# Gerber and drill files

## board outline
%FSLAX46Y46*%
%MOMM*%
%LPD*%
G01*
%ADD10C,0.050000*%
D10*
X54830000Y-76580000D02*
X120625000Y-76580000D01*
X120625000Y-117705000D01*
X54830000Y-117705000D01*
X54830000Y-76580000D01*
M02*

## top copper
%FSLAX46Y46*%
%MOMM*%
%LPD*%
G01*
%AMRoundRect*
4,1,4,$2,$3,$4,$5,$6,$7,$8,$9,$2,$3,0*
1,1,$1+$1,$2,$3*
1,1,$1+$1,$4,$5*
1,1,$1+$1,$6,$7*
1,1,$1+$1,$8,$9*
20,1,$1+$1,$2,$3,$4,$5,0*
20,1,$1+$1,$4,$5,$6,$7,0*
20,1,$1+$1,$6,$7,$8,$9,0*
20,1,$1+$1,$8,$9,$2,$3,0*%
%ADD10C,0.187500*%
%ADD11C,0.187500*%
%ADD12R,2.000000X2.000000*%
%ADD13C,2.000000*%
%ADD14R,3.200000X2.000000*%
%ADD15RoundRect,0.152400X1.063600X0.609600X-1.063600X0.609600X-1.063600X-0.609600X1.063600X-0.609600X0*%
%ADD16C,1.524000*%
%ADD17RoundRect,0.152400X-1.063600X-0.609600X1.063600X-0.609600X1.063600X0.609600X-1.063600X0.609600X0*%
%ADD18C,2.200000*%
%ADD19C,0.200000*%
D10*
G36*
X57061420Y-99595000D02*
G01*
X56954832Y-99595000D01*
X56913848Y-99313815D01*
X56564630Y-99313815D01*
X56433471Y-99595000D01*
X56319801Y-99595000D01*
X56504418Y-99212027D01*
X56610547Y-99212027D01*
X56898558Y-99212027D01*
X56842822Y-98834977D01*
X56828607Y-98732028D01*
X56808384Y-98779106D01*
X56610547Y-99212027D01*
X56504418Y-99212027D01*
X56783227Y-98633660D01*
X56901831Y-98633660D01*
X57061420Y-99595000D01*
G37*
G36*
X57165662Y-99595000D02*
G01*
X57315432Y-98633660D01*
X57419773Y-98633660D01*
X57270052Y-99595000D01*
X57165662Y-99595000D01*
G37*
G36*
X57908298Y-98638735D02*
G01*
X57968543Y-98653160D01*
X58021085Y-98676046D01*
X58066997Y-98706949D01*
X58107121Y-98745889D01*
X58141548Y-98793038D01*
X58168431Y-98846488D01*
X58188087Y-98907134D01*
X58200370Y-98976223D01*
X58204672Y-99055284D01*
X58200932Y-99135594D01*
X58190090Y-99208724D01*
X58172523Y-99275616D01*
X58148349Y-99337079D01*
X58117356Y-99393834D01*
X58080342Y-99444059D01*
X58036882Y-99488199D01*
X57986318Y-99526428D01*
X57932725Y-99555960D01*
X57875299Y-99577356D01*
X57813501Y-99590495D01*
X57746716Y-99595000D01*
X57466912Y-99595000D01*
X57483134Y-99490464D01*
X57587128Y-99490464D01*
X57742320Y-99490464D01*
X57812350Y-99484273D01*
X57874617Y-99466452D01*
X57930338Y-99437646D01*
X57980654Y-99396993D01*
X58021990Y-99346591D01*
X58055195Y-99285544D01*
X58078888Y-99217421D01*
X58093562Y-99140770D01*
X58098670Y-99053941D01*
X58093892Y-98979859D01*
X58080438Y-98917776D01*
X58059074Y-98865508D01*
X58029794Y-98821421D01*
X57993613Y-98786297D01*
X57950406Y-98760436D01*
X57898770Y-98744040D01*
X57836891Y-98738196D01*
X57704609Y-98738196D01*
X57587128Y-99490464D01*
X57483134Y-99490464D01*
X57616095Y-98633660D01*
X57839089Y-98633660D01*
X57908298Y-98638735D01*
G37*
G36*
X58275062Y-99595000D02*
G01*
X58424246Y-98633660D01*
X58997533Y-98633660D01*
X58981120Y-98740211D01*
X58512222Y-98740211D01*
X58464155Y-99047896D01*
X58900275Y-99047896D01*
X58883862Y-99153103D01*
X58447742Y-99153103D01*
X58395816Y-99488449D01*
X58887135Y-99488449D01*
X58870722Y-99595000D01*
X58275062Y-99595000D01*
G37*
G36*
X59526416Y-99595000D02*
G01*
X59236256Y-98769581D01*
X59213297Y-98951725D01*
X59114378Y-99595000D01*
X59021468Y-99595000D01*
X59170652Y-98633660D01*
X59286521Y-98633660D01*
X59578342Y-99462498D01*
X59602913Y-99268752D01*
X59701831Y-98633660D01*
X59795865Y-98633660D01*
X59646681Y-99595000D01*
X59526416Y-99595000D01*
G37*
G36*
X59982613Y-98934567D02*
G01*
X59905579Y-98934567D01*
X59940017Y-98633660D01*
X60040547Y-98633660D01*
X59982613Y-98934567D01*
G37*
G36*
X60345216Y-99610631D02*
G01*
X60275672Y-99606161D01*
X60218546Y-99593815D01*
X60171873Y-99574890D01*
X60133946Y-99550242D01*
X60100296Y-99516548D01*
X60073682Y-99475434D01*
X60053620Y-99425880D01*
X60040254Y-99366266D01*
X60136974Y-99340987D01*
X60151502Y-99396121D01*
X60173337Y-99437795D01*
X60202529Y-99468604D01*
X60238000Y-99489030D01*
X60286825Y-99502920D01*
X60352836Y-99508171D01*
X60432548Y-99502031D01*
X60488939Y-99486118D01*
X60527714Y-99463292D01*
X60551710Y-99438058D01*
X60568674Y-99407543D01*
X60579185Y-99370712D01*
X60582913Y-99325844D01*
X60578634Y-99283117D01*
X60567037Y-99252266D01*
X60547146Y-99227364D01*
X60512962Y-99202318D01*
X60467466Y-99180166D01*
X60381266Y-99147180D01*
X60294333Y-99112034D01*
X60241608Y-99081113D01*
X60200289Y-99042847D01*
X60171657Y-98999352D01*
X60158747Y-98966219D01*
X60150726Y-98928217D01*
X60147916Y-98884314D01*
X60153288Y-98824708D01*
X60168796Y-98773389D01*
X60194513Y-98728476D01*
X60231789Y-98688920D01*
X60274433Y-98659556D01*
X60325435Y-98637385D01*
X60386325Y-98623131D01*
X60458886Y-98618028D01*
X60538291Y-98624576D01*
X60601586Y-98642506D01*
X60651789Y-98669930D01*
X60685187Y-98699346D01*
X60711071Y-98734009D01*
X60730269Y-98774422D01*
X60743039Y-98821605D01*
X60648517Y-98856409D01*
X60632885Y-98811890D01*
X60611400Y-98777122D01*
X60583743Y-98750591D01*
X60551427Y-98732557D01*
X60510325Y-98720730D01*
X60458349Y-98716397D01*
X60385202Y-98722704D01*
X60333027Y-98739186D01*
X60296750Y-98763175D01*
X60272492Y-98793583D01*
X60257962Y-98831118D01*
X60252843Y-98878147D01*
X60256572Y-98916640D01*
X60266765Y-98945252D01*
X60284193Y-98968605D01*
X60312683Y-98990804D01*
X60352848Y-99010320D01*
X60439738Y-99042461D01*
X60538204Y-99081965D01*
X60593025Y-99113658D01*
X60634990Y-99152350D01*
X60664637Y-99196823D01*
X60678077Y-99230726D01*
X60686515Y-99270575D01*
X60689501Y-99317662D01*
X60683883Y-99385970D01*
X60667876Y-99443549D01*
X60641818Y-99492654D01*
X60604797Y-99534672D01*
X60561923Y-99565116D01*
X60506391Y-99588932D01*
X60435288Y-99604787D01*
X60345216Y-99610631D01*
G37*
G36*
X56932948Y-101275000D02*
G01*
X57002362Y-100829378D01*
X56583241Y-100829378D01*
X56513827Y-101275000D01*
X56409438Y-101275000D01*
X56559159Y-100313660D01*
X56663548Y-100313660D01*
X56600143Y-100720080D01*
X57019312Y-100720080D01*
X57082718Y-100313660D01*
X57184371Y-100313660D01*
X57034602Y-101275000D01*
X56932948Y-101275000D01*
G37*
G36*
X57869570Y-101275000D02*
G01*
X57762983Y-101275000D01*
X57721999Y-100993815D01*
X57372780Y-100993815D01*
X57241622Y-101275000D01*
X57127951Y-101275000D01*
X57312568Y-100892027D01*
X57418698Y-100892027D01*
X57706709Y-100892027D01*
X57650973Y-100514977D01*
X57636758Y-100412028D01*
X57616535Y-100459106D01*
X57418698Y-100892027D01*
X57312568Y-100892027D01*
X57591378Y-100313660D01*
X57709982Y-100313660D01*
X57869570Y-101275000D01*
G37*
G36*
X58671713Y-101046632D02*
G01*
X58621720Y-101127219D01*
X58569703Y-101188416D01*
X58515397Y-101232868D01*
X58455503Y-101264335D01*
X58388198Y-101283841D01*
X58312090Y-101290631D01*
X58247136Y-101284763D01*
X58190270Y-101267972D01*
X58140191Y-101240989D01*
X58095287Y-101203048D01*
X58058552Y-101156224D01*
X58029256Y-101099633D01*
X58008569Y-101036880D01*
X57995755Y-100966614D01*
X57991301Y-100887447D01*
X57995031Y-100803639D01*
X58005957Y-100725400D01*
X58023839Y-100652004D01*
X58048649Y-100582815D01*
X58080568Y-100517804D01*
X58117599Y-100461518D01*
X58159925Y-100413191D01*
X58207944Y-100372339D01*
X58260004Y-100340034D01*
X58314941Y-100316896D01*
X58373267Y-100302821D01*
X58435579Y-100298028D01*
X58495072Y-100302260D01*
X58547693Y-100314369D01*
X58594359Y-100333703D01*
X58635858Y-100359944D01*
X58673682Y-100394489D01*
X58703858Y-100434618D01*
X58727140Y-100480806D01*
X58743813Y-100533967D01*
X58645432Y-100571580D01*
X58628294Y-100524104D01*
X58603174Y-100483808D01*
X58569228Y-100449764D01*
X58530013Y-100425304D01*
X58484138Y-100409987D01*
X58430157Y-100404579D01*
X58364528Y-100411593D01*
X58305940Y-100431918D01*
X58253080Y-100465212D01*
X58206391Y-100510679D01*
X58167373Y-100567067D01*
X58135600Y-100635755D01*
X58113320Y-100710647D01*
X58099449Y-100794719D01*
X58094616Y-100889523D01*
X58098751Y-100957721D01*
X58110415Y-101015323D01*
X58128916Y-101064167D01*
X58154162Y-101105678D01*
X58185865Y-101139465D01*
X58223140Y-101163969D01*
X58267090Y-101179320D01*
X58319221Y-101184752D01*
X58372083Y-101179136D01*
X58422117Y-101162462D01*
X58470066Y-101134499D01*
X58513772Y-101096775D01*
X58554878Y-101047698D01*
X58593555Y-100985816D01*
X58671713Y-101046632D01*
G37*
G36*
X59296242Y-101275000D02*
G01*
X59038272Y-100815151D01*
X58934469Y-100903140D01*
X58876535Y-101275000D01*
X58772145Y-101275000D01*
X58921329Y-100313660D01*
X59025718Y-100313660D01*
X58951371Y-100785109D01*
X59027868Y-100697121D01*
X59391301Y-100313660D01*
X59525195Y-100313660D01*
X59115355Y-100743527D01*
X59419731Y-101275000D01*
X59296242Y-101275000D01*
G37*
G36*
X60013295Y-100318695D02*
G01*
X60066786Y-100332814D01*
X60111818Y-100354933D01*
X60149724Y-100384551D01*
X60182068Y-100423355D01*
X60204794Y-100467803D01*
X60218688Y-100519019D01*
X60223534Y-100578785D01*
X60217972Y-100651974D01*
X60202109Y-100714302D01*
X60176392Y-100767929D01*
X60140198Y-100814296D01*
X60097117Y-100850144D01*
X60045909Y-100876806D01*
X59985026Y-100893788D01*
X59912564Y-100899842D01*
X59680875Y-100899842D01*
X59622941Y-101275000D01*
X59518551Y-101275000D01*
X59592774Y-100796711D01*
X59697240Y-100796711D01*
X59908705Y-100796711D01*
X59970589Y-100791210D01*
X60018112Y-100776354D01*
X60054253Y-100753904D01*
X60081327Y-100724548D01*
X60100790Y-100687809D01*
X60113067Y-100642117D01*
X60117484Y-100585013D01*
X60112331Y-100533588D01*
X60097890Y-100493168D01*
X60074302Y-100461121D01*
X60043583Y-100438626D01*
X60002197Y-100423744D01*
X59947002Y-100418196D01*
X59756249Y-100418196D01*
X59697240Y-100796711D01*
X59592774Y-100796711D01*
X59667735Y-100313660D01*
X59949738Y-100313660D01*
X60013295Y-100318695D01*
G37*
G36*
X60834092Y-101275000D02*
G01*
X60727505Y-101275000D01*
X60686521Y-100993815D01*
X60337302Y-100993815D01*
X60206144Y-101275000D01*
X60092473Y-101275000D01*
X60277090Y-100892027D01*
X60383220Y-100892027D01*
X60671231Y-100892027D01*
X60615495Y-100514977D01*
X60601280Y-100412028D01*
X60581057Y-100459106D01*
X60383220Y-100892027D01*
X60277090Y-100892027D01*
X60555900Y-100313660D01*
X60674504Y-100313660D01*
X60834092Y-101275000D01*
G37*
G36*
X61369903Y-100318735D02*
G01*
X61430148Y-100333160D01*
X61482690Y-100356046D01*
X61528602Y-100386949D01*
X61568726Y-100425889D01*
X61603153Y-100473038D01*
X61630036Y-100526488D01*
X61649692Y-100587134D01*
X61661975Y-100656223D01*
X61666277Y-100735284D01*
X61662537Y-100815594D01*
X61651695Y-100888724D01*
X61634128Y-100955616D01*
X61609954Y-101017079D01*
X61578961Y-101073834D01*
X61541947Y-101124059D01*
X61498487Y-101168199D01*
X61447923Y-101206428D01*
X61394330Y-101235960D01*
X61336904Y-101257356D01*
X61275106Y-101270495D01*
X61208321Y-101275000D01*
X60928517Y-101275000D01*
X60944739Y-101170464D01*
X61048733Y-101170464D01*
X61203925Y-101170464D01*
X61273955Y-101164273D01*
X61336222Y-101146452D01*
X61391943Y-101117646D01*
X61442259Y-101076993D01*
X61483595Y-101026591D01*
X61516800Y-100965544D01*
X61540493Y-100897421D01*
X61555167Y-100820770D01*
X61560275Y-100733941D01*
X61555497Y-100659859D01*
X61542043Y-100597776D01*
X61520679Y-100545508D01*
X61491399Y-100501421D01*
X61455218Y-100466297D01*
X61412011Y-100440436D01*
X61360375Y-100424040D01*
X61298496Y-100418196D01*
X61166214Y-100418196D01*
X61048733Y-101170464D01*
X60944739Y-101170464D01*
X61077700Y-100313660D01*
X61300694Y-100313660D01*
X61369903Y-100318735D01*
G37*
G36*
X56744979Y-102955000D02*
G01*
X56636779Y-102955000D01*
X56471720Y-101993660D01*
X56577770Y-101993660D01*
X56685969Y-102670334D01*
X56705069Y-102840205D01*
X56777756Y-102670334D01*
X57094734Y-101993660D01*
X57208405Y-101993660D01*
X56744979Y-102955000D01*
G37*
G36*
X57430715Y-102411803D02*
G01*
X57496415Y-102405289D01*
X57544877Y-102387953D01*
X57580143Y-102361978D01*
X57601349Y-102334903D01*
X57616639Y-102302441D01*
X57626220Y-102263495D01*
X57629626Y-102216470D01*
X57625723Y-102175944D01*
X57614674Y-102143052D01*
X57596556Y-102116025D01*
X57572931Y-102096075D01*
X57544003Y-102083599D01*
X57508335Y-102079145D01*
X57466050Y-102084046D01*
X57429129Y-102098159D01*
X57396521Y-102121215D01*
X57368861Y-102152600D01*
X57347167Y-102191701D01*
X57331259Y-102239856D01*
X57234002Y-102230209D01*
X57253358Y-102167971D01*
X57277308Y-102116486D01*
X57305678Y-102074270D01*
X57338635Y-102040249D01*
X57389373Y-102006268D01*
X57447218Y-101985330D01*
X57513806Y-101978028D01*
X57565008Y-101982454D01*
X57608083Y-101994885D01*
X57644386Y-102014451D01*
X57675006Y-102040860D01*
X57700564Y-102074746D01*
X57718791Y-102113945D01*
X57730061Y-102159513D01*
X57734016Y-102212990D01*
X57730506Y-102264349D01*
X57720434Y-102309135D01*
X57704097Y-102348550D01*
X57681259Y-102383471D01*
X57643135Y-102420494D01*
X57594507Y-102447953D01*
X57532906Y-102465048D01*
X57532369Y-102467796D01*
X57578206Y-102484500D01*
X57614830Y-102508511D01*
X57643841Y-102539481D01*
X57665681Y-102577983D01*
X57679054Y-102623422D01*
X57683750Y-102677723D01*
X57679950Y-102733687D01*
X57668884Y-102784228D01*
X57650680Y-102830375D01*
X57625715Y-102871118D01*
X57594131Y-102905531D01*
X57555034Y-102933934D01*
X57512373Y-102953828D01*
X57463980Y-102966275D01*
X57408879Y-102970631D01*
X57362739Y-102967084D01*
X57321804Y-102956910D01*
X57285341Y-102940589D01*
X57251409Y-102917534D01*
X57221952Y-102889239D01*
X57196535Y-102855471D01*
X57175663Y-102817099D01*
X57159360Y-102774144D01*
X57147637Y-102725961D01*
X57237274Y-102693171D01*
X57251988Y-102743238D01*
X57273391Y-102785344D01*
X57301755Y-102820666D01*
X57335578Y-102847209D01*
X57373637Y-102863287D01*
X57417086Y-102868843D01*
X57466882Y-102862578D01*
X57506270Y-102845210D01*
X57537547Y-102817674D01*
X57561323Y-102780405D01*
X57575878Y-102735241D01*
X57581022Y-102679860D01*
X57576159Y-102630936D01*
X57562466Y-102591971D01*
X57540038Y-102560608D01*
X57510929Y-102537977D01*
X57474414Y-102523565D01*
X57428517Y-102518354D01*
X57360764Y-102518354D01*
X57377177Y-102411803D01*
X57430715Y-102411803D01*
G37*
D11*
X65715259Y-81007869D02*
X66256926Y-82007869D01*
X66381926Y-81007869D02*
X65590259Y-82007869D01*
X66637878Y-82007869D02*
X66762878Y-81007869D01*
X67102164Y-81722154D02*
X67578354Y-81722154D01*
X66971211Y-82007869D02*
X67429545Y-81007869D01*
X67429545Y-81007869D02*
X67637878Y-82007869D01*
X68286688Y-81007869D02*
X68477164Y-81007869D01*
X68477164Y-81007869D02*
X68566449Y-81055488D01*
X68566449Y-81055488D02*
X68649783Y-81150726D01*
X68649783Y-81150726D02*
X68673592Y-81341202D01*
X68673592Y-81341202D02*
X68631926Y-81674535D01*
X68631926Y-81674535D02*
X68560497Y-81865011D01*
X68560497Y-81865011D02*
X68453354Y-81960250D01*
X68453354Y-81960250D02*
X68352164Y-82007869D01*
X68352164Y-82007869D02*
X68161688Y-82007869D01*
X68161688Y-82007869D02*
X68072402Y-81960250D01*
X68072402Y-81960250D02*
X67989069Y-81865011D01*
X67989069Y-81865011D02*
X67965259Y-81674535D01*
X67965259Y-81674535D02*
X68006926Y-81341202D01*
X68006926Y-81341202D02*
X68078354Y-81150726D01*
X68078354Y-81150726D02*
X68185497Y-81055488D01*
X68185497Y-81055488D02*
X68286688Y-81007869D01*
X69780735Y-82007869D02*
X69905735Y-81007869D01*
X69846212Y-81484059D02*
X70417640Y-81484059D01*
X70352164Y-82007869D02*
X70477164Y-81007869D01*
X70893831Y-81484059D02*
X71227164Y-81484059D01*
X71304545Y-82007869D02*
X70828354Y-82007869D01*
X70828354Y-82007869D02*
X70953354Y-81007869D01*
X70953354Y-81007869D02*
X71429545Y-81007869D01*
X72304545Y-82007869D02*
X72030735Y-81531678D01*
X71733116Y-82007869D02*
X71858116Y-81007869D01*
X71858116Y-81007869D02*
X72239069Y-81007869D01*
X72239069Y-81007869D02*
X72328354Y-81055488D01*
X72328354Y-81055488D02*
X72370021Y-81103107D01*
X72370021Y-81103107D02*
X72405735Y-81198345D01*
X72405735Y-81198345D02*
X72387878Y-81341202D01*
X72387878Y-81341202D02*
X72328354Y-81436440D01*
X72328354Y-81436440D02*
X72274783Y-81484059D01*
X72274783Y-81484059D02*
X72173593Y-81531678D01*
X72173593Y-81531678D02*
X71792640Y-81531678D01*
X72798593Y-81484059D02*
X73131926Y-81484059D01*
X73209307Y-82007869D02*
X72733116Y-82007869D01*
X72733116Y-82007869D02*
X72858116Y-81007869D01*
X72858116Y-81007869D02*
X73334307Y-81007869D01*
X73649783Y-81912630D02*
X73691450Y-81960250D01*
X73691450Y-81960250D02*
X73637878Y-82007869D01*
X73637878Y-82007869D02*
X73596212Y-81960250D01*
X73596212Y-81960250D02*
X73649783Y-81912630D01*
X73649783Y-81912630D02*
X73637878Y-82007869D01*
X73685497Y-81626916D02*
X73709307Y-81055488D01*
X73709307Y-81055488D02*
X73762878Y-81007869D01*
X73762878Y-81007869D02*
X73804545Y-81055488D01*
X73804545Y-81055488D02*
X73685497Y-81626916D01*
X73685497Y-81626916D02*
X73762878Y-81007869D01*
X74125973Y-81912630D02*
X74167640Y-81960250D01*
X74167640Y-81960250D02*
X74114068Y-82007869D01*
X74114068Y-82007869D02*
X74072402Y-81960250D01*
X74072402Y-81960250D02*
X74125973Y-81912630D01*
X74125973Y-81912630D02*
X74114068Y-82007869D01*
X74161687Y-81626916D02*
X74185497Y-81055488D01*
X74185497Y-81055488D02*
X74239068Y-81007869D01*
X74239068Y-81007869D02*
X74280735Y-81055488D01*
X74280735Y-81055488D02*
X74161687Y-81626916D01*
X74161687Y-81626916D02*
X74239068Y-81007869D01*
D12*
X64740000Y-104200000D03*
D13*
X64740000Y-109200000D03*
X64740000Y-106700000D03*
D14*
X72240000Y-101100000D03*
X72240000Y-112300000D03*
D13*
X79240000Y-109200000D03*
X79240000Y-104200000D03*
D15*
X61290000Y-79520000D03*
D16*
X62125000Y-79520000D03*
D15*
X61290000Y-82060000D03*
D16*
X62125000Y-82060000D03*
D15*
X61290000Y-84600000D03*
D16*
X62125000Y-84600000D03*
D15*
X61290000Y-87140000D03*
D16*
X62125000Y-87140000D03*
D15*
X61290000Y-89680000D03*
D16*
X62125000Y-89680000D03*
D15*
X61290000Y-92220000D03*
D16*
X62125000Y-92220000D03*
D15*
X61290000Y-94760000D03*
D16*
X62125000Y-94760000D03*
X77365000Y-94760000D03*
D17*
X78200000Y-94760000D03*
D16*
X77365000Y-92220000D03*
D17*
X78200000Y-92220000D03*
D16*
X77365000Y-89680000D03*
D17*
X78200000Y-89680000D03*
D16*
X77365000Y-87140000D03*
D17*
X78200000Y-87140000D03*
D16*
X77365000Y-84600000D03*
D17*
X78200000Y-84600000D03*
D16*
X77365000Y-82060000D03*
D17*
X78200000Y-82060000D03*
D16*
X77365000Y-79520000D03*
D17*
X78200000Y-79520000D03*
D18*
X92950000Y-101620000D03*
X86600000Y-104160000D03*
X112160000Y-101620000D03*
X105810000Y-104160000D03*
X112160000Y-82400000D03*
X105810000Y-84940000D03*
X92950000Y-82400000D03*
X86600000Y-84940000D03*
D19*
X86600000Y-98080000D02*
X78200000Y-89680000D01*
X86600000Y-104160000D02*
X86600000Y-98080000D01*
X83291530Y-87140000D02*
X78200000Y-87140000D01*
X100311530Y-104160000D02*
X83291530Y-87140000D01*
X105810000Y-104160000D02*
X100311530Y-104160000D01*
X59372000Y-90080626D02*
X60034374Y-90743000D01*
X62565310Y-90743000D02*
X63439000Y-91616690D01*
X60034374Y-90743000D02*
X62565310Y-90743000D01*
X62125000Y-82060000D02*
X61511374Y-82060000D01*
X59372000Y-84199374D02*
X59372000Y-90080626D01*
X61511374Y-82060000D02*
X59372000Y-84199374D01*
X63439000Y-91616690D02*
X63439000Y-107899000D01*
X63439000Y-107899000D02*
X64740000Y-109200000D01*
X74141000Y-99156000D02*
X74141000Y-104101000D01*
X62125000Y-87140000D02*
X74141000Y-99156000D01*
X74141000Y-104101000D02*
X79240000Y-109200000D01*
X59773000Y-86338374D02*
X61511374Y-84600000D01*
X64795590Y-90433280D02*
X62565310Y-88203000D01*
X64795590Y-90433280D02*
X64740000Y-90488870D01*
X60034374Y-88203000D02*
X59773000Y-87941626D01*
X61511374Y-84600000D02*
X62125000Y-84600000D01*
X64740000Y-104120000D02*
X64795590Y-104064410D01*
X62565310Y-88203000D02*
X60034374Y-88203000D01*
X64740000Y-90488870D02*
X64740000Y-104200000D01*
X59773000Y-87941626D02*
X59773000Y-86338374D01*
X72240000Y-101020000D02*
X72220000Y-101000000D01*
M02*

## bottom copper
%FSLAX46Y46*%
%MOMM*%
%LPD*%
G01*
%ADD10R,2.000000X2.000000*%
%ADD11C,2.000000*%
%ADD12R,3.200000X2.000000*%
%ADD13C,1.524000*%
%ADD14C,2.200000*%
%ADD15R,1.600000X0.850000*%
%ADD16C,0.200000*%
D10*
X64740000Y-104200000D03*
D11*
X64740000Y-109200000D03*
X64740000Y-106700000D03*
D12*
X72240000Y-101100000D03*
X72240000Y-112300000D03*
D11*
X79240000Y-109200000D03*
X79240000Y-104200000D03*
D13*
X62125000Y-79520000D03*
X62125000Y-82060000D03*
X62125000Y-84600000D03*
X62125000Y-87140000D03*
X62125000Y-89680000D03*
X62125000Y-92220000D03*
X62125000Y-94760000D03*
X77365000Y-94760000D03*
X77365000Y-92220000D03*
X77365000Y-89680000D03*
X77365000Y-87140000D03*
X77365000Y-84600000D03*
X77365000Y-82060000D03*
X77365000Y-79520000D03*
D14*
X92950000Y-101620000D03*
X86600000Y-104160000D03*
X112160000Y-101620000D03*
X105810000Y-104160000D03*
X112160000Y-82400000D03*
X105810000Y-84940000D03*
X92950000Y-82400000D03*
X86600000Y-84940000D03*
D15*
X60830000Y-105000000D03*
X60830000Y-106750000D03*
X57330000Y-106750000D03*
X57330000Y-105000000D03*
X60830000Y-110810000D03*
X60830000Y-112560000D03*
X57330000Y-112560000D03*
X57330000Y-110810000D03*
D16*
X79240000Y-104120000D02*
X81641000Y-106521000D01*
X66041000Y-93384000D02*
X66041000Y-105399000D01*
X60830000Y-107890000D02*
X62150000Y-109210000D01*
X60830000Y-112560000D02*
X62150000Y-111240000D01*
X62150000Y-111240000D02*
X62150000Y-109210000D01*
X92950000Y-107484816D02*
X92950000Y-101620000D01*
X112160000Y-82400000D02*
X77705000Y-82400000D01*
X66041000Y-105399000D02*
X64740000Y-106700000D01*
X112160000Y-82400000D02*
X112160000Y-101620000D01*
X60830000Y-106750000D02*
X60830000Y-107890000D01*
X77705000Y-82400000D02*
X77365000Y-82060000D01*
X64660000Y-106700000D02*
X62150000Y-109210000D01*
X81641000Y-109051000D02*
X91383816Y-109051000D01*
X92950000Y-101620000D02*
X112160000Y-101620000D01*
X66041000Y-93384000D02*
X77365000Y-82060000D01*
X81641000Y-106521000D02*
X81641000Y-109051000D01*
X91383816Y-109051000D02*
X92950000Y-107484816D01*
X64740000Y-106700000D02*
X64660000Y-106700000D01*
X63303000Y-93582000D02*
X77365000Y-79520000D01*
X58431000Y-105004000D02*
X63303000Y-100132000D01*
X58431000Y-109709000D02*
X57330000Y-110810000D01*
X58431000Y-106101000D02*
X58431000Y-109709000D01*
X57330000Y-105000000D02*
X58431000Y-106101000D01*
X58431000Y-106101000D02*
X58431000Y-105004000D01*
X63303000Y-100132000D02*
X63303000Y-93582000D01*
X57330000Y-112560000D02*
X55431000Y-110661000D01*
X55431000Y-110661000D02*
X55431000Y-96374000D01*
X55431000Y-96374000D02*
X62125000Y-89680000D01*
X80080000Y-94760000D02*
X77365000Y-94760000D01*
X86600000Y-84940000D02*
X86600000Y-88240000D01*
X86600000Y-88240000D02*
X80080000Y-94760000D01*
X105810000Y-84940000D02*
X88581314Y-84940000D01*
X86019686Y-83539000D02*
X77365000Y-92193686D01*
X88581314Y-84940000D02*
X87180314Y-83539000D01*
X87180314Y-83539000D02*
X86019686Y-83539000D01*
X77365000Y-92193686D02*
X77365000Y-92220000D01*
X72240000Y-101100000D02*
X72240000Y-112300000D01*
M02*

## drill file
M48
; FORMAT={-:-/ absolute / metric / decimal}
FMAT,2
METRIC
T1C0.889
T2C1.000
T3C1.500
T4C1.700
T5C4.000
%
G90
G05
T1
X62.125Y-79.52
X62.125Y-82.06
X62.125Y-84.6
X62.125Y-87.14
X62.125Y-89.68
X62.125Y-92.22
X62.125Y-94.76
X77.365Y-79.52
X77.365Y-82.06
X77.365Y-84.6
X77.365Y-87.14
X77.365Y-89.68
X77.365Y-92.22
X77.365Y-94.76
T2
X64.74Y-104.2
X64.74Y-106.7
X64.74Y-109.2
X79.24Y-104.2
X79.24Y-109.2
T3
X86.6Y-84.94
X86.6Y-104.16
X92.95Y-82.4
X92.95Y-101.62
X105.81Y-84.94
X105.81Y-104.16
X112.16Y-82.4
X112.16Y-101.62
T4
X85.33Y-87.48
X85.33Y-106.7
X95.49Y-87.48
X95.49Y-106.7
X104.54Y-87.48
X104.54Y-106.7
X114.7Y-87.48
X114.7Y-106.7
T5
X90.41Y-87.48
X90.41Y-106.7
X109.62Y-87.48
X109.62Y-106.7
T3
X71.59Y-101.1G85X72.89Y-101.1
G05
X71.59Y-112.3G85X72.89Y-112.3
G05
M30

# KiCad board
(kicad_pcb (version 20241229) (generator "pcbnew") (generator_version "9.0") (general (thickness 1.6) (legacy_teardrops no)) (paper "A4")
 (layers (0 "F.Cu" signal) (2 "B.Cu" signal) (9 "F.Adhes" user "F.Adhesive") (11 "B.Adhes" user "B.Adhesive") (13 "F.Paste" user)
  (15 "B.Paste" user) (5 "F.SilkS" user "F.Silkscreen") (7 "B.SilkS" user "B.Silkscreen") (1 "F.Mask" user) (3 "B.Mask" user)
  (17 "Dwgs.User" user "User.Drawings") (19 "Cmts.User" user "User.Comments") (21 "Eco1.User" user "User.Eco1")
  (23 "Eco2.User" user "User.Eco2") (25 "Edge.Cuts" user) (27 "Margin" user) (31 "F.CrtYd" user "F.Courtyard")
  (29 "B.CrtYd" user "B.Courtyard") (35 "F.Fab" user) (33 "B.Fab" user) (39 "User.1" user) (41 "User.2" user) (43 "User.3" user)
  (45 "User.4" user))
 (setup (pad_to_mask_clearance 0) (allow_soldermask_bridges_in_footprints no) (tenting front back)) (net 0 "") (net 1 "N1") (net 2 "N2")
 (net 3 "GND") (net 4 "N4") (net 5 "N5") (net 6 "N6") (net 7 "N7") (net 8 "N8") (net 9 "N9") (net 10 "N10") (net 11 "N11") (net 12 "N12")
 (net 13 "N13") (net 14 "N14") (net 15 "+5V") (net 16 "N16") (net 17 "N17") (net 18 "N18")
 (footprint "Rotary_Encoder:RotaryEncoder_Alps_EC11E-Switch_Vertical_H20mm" (layer "F.Cu") (at 64.74 104.2)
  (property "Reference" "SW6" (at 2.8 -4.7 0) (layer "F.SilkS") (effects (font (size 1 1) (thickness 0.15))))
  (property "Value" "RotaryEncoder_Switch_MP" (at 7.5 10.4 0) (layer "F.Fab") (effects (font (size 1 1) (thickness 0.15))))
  (pad "A" thru_hole rect (at 0 0) (size 2 2) (drill 1) (layers "*.Cu" "*.Mask") (remove_unused_layers no) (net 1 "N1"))
  (pad "B" thru_hole circle (at 0 5) (size 2 2) (drill 1) (layers "*.Cu" "*.Mask") (remove_unused_layers no) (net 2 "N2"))
  (pad "C" thru_hole circle (at 0 2.5) (size 2 2) (drill 1) (layers "*.Cu" "*.Mask") (remove_unused_layers no) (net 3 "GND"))
  (pad "MP" thru_hole rect (at 7.5 -3.1) (size 3.2 2) (drill oval 2.8 1.5) (layers "*.Cu" "*.Mask") (remove_unused_layers no) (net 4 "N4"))
  (pad "MP" thru_hole rect (at 7.5 8.1) (size 3.2 2) (drill oval 2.8 1.5) (layers "*.Cu" "*.Mask") (remove_unused_layers no) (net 4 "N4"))
  (pad "S1" thru_hole circle (at 14.5 5) (size 2 2) (drill 1) (layers "*.Cu" "*.Mask") (remove_unused_layers no) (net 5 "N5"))
  (pad "S2" thru_hole circle (at 14.5 0) (size 2 2) (drill 1) (layers "*.Cu" "*.Mask") (remove_unused_layers no) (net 3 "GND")))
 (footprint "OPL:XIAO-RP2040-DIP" (layer "F.Cu") (at 69.745 87.14)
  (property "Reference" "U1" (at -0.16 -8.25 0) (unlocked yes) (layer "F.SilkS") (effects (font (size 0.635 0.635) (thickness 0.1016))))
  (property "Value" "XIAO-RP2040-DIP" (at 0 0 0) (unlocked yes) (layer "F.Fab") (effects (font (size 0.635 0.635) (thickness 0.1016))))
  (pad "1" smd roundrect (at -8.455 -7.62 180) (size 2.432 1.524) (layers "F.Cu" "F.Mask") (roundrect_rratio 0.1) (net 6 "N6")
   (thermal_bridge_angle 45))
  (pad "1" thru_hole circle (at -7.62 -7.62 180) (size 1.524 1.524) (drill 0.889) (layers "*.Cu" "*.Mask") (remove_unused_layers no)
   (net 6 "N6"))
  (pad "2" smd roundrect (at -8.455 -5.08 180) (size 2.432 1.524) (layers "F.Cu" "F.Mask") (roundrect_rratio 0.1) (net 2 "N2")
   (thermal_bridge_angle 45))
  (pad "2" thru_hole circle (at -7.62 -5.08 180) (size 1.524 1.524) (drill 0.889) (layers "*.Cu" "*.Mask") (remove_unused_layers no)
   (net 2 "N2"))
  (pad "3" smd roundrect (at -8.455 -2.54 180) (size 2.432 1.524) (layers "F.Cu" "F.Mask") (roundrect_rratio 0.1) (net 1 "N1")
   (thermal_bridge_angle 45))
  (pad "3" thru_hole circle (at -7.62 -2.54 180) (size 1.524 1.524) (drill 0.889) (layers "*.Cu" "*.Mask") (remove_unused_layers no)
   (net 1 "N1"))
  (pad "4" smd roundrect (at -8.455 0 180) (size 2.432 1.524) (layers "F.Cu" "F.Mask") (roundrect_rratio 0.1) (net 5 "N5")
   (thermal_bridge_angle 45))
  (pad "4" thru_hole circle (at -7.62 0 180) (size 1.524 1.524) (drill 0.889) (layers "*.Cu" "*.Mask") (remove_unused_layers no)
   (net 5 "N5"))
  (pad "5" smd roundrect (at -8.455 2.54 180) (size 2.432 1.524) (layers "F.Cu" "F.Mask") (roundrect_rratio 0.1) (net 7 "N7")
   (thermal_bridge_angle 45))
  (pad "5" thru_hole circle (at -7.62 2.54 180) (size 1.524 1.524) (drill 0.889) (layers "*.Cu" "*.Mask") (remove_unused_layers no)
   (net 7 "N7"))
  (pad "6" smd roundrect (at -8.455 5.08 180) (size 2.432 1.524) (layers "F.Cu" "F.Mask") (roundrect_rratio 0.1) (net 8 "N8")
   (thermal_bridge_angle 45))
  (pad "6" thru_hole circle (at -7.62 5.08 180) (size 1.524 1.524) (drill 0.889) (layers "*.Cu" "*.Mask") (remove_unused_layers no)
   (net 8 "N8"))
  (pad "7" smd roundrect (at -8.455 7.62 180) (size 2.432 1.524) (layers "F.Cu" "F.Mask") (roundrect_rratio 0.1) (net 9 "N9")
   (thermal_bridge_angle 45))
  (pad "7" thru_hole circle (at -7.62 7.62 180) (size 1.524 1.524) (drill 0.889) (layers "*.Cu" "*.Mask") (remove_unused_layers no)
   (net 9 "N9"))
  (pad "8" thru_hole circle (at 7.62 7.62) (size 1.524 1.524) (drill 0.889) (layers "*.Cu" "*.Mask") (remove_unused_layers no)
   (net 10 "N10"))
  (pad "8" smd roundrect (at 8.455 7.62) (size 2.432 1.524) (layers "F.Cu" "F.Mask") (roundrect_rratio 0.1) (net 10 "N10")
   (thermal_bridge_angle 45))
  (pad "9" thru_hole circle (at 7.62 5.08) (size 1.524 1.524) (drill 0.889) (layers "*.Cu" "*.Mask") (remove_unused_layers no)
   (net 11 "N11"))
  (pad "9" smd roundrect (at 8.455 5.08) (size 2.432 1.524) (layers "F.Cu" "F.Mask") (roundrect_rratio 0.1) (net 11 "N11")
   (thermal_bridge_angle 45))
  (pad "10" thru_hole circle (at 7.62 2.54) (size 1.524 1.524) (drill 0.889) (layers "*.Cu" "*.Mask") (remove_unused_layers no)
   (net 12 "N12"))
  (pad "10" smd roundrect (at 8.455 2.54) (size 2.432 1.524) (layers "F.Cu" "F.Mask") (roundrect_rratio 0.1) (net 12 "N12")
   (thermal_bridge_angle 45))
  (pad "11" thru_hole circle (at 7.62 0) (size 1.524 1.524) (drill 0.889) (layers "*.Cu" "*.Mask") (remove_unused_layers no) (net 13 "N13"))
  (pad "11" smd roundrect (at 8.455 0) (size 2.432 1.524) (layers "F.Cu" "F.Mask") (roundrect_rratio 0.1) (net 13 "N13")
   (thermal_bridge_angle 45))
  (pad "12" thru_hole circle (at 7.62 -2.54) (size 1.524 1.524) (drill 0.889) (layers "*.Cu" "*.Mask") (remove_unused_layers no)
   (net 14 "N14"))
  (pad "12" smd roundrect (at 8.455 -2.54) (size 2.432 1.524) (layers "F.Cu" "F.Mask") (roundrect_rratio 0.1) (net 14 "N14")
   (thermal_bridge_angle 45))
  (pad "13" thru_hole circle (at 7.62 -5.08) (size 1.524 1.524) (drill 0.889) (layers "*.Cu" "*.Mask") (remove_unused_layers no)
   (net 3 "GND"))
  (pad "13" smd roundrect (at 8.455 -5.08) (size 2.432 1.524) (layers "F.Cu" "F.Mask") (roundrect_rratio 0.1) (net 3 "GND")
   (thermal_bridge_angle 45))
  (pad "14" thru_hole circle (at 7.62 -7.62) (size 1.524 1.524) (drill 0.889) (layers "*.Cu" "*.Mask") (remove_unused_layers no)
   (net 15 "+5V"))
  (pad "14" smd roundrect (at 8.455 -7.62) (size 2.432 1.524) (layers "F.Cu" "F.Mask") (roundrect_rratio 0.1) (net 15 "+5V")
   (thermal_bridge_angle 45)))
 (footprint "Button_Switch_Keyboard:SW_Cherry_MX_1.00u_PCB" (layer "F.Cu") (at 92.95 101.62)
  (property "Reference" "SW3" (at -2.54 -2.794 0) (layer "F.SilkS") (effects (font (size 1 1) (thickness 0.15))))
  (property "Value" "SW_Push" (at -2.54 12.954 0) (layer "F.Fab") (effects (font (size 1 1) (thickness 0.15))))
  (pad "" np_thru_hole circle (at -7.62 5.08) (size 1.7 1.7) (drill 1.7) (layers "*.Cu" "*.Mask"))
  (pad "" np_thru_hole circle (at -2.54 5.08) (size 4 4) (drill 4) (layers "*.Cu" "*.Mask"))
  (pad "" np_thru_hole circle (at 2.54 5.08) (size 1.7 1.7) (drill 1.7) (layers "*.Cu" "*.Mask"))
  (pad "1" thru_hole circle (at 0 0) (size 2.2 2.2) (drill 1.5) (layers "*.Cu" "*.Mask") (remove_unused_layers no) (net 3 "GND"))
  (pad "2" thru_hole circle (at -6.35 2.54) (size 2.2 2.2) (drill 1.5) (layers "*.Cu" "*.Mask") (remove_unused_layers no) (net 12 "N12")))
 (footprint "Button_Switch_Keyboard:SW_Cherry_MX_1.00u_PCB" (layer "F.Cu") (at 112.16 101.62)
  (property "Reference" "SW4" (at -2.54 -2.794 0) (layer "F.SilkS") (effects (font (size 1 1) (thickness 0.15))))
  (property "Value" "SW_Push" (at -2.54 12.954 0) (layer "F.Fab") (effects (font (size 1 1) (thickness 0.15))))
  (pad "" np_thru_hole circle (at -7.62 5.08) (size 1.7 1.7) (drill 1.7) (layers "*.Cu" "*.Mask"))
  (pad "" np_thru_hole circle (at -2.54 5.08) (size 4 4) (drill 4) (layers "*.Cu" "*.Mask"))
  (pad "" np_thru_hole circle (at 2.54 5.08) (size 1.7 1.7) (drill 1.7) (layers "*.Cu" "*.Mask"))
  (pad "1" thru_hole circle (at 0 0) (size 2.2 2.2) (drill 1.5) (layers "*.Cu" "*.Mask") (remove_unused_layers no) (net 3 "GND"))
  (pad "2" thru_hole circle (at -6.35 2.54) (size 2.2 2.2) (drill 1.5) (layers "*.Cu" "*.Mask") (remove_unused_layers no) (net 13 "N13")))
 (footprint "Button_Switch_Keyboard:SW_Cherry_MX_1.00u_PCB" (layer "F.Cu") (at 112.16 82.4)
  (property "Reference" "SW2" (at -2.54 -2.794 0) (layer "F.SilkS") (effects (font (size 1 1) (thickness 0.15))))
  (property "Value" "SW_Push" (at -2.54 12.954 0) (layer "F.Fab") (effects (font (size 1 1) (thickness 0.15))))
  (pad "" np_thru_hole circle (at -7.62 5.08) (size 1.7 1.7) (drill 1.7) (layers "*.Cu" "*.Mask"))
  (pad "" np_thru_hole circle (at -2.54 5.08) (size 4 4) (drill 4) (layers "*.Cu" "*.Mask"))
  (pad "" np_thru_hole circle (at 2.54 5.08) (size 1.7 1.7) (drill 1.7) (layers "*.Cu" "*.Mask"))
  (pad "1" thru_hole circle (at 0 0) (size 2.2 2.2) (drill 1.5) (layers "*.Cu" "*.Mask") (remove_unused_layers no) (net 3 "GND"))
  (pad "2" thru_hole circle (at -6.35 2.54) (size 2.2 2.2) (drill 1.5) (layers "*.Cu" "*.Mask") (remove_unused_layers no) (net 11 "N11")))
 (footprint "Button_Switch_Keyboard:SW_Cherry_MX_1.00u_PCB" (layer "F.Cu") (at 92.95 82.4)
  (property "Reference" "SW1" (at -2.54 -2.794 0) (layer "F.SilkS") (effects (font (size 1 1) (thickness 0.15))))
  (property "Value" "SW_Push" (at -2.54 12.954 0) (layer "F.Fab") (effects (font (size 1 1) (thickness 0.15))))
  (pad "" np_thru_hole circle (at -7.62 5.08) (size 1.7 1.7) (drill 1.7) (layers "*.Cu" "*.Mask"))
  (pad "" np_thru_hole circle (at -2.54 5.08) (size 4 4) (drill 4) (layers "*.Cu" "*.Mask"))
  (pad "" np_thru_hole circle (at 2.54 5.08) (size 1.7 1.7) (drill 1.7) (layers "*.Cu" "*.Mask"))
  (pad "1" thru_hole circle (at 0 0) (size 2.2 2.2) (drill 1.5) (layers "*.Cu" "*.Mask") (remove_unused_layers no) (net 3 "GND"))
  (pad "2" thru_hole circle (at -6.35 2.54) (size 2.2 2.2) (drill 1.5) (layers "*.Cu" "*.Mask") (remove_unused_layers no) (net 10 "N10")))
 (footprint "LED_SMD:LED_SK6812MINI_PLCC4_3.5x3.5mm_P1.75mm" (layer "B.Cu") (at 59.08 105.875 180)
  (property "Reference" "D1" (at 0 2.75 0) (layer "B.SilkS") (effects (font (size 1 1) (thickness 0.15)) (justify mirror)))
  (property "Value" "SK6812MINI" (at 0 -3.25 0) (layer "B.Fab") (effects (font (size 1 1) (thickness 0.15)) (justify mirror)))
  (pad "1" smd rect (at -1.75 0.875 180) (size 1.6 0.85) (layers "B.Cu" "B.Mask" "B.Paste") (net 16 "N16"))
  (pad "2" smd rect (at -1.75 -0.875 180) (size 1.6 0.85) (layers "B.Cu" "B.Mask" "B.Paste") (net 3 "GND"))
  (pad "3" smd rect (at 1.75 -0.875 180) (size 1.6 0.85) (layers "B.Cu" "B.Mask" "B.Paste") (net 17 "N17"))
  (pad "4" smd rect (at 1.75 0.875 180) (size 1.6 0.85) (layers "B.Cu" "B.Mask" "B.Paste") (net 15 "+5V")))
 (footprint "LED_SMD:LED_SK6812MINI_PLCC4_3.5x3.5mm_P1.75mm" (layer "B.Cu") (at 59.08 111.685 180)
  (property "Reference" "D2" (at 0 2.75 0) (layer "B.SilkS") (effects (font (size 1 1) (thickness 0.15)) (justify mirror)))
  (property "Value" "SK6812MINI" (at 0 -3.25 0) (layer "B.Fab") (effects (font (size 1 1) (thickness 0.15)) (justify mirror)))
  (pad "1" smd rect (at -1.75 0.875 180) (size 1.6 0.85) (layers "B.Cu" "B.Mask" "B.Paste") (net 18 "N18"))
  (pad "2" smd rect (at -1.75 -0.875 180) (size 1.6 0.85) (layers "B.Cu" "B.Mask" "B.Paste") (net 3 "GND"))
  (pad "3" smd rect (at 1.75 -0.875 180) (size 1.6 0.85) (layers "B.Cu" "B.Mask" "B.Paste") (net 7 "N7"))
  (pad "4" smd rect (at 1.75 0.875 180) (size 1.6 0.85) (layers "B.Cu" "B.Mask" "B.Paste") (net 15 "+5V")))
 (gr_rect (start 54.83 76.58) (end 120.625 117.705) (stroke (width 0.05) (type default)) (fill no) (layer "Edge.Cuts"))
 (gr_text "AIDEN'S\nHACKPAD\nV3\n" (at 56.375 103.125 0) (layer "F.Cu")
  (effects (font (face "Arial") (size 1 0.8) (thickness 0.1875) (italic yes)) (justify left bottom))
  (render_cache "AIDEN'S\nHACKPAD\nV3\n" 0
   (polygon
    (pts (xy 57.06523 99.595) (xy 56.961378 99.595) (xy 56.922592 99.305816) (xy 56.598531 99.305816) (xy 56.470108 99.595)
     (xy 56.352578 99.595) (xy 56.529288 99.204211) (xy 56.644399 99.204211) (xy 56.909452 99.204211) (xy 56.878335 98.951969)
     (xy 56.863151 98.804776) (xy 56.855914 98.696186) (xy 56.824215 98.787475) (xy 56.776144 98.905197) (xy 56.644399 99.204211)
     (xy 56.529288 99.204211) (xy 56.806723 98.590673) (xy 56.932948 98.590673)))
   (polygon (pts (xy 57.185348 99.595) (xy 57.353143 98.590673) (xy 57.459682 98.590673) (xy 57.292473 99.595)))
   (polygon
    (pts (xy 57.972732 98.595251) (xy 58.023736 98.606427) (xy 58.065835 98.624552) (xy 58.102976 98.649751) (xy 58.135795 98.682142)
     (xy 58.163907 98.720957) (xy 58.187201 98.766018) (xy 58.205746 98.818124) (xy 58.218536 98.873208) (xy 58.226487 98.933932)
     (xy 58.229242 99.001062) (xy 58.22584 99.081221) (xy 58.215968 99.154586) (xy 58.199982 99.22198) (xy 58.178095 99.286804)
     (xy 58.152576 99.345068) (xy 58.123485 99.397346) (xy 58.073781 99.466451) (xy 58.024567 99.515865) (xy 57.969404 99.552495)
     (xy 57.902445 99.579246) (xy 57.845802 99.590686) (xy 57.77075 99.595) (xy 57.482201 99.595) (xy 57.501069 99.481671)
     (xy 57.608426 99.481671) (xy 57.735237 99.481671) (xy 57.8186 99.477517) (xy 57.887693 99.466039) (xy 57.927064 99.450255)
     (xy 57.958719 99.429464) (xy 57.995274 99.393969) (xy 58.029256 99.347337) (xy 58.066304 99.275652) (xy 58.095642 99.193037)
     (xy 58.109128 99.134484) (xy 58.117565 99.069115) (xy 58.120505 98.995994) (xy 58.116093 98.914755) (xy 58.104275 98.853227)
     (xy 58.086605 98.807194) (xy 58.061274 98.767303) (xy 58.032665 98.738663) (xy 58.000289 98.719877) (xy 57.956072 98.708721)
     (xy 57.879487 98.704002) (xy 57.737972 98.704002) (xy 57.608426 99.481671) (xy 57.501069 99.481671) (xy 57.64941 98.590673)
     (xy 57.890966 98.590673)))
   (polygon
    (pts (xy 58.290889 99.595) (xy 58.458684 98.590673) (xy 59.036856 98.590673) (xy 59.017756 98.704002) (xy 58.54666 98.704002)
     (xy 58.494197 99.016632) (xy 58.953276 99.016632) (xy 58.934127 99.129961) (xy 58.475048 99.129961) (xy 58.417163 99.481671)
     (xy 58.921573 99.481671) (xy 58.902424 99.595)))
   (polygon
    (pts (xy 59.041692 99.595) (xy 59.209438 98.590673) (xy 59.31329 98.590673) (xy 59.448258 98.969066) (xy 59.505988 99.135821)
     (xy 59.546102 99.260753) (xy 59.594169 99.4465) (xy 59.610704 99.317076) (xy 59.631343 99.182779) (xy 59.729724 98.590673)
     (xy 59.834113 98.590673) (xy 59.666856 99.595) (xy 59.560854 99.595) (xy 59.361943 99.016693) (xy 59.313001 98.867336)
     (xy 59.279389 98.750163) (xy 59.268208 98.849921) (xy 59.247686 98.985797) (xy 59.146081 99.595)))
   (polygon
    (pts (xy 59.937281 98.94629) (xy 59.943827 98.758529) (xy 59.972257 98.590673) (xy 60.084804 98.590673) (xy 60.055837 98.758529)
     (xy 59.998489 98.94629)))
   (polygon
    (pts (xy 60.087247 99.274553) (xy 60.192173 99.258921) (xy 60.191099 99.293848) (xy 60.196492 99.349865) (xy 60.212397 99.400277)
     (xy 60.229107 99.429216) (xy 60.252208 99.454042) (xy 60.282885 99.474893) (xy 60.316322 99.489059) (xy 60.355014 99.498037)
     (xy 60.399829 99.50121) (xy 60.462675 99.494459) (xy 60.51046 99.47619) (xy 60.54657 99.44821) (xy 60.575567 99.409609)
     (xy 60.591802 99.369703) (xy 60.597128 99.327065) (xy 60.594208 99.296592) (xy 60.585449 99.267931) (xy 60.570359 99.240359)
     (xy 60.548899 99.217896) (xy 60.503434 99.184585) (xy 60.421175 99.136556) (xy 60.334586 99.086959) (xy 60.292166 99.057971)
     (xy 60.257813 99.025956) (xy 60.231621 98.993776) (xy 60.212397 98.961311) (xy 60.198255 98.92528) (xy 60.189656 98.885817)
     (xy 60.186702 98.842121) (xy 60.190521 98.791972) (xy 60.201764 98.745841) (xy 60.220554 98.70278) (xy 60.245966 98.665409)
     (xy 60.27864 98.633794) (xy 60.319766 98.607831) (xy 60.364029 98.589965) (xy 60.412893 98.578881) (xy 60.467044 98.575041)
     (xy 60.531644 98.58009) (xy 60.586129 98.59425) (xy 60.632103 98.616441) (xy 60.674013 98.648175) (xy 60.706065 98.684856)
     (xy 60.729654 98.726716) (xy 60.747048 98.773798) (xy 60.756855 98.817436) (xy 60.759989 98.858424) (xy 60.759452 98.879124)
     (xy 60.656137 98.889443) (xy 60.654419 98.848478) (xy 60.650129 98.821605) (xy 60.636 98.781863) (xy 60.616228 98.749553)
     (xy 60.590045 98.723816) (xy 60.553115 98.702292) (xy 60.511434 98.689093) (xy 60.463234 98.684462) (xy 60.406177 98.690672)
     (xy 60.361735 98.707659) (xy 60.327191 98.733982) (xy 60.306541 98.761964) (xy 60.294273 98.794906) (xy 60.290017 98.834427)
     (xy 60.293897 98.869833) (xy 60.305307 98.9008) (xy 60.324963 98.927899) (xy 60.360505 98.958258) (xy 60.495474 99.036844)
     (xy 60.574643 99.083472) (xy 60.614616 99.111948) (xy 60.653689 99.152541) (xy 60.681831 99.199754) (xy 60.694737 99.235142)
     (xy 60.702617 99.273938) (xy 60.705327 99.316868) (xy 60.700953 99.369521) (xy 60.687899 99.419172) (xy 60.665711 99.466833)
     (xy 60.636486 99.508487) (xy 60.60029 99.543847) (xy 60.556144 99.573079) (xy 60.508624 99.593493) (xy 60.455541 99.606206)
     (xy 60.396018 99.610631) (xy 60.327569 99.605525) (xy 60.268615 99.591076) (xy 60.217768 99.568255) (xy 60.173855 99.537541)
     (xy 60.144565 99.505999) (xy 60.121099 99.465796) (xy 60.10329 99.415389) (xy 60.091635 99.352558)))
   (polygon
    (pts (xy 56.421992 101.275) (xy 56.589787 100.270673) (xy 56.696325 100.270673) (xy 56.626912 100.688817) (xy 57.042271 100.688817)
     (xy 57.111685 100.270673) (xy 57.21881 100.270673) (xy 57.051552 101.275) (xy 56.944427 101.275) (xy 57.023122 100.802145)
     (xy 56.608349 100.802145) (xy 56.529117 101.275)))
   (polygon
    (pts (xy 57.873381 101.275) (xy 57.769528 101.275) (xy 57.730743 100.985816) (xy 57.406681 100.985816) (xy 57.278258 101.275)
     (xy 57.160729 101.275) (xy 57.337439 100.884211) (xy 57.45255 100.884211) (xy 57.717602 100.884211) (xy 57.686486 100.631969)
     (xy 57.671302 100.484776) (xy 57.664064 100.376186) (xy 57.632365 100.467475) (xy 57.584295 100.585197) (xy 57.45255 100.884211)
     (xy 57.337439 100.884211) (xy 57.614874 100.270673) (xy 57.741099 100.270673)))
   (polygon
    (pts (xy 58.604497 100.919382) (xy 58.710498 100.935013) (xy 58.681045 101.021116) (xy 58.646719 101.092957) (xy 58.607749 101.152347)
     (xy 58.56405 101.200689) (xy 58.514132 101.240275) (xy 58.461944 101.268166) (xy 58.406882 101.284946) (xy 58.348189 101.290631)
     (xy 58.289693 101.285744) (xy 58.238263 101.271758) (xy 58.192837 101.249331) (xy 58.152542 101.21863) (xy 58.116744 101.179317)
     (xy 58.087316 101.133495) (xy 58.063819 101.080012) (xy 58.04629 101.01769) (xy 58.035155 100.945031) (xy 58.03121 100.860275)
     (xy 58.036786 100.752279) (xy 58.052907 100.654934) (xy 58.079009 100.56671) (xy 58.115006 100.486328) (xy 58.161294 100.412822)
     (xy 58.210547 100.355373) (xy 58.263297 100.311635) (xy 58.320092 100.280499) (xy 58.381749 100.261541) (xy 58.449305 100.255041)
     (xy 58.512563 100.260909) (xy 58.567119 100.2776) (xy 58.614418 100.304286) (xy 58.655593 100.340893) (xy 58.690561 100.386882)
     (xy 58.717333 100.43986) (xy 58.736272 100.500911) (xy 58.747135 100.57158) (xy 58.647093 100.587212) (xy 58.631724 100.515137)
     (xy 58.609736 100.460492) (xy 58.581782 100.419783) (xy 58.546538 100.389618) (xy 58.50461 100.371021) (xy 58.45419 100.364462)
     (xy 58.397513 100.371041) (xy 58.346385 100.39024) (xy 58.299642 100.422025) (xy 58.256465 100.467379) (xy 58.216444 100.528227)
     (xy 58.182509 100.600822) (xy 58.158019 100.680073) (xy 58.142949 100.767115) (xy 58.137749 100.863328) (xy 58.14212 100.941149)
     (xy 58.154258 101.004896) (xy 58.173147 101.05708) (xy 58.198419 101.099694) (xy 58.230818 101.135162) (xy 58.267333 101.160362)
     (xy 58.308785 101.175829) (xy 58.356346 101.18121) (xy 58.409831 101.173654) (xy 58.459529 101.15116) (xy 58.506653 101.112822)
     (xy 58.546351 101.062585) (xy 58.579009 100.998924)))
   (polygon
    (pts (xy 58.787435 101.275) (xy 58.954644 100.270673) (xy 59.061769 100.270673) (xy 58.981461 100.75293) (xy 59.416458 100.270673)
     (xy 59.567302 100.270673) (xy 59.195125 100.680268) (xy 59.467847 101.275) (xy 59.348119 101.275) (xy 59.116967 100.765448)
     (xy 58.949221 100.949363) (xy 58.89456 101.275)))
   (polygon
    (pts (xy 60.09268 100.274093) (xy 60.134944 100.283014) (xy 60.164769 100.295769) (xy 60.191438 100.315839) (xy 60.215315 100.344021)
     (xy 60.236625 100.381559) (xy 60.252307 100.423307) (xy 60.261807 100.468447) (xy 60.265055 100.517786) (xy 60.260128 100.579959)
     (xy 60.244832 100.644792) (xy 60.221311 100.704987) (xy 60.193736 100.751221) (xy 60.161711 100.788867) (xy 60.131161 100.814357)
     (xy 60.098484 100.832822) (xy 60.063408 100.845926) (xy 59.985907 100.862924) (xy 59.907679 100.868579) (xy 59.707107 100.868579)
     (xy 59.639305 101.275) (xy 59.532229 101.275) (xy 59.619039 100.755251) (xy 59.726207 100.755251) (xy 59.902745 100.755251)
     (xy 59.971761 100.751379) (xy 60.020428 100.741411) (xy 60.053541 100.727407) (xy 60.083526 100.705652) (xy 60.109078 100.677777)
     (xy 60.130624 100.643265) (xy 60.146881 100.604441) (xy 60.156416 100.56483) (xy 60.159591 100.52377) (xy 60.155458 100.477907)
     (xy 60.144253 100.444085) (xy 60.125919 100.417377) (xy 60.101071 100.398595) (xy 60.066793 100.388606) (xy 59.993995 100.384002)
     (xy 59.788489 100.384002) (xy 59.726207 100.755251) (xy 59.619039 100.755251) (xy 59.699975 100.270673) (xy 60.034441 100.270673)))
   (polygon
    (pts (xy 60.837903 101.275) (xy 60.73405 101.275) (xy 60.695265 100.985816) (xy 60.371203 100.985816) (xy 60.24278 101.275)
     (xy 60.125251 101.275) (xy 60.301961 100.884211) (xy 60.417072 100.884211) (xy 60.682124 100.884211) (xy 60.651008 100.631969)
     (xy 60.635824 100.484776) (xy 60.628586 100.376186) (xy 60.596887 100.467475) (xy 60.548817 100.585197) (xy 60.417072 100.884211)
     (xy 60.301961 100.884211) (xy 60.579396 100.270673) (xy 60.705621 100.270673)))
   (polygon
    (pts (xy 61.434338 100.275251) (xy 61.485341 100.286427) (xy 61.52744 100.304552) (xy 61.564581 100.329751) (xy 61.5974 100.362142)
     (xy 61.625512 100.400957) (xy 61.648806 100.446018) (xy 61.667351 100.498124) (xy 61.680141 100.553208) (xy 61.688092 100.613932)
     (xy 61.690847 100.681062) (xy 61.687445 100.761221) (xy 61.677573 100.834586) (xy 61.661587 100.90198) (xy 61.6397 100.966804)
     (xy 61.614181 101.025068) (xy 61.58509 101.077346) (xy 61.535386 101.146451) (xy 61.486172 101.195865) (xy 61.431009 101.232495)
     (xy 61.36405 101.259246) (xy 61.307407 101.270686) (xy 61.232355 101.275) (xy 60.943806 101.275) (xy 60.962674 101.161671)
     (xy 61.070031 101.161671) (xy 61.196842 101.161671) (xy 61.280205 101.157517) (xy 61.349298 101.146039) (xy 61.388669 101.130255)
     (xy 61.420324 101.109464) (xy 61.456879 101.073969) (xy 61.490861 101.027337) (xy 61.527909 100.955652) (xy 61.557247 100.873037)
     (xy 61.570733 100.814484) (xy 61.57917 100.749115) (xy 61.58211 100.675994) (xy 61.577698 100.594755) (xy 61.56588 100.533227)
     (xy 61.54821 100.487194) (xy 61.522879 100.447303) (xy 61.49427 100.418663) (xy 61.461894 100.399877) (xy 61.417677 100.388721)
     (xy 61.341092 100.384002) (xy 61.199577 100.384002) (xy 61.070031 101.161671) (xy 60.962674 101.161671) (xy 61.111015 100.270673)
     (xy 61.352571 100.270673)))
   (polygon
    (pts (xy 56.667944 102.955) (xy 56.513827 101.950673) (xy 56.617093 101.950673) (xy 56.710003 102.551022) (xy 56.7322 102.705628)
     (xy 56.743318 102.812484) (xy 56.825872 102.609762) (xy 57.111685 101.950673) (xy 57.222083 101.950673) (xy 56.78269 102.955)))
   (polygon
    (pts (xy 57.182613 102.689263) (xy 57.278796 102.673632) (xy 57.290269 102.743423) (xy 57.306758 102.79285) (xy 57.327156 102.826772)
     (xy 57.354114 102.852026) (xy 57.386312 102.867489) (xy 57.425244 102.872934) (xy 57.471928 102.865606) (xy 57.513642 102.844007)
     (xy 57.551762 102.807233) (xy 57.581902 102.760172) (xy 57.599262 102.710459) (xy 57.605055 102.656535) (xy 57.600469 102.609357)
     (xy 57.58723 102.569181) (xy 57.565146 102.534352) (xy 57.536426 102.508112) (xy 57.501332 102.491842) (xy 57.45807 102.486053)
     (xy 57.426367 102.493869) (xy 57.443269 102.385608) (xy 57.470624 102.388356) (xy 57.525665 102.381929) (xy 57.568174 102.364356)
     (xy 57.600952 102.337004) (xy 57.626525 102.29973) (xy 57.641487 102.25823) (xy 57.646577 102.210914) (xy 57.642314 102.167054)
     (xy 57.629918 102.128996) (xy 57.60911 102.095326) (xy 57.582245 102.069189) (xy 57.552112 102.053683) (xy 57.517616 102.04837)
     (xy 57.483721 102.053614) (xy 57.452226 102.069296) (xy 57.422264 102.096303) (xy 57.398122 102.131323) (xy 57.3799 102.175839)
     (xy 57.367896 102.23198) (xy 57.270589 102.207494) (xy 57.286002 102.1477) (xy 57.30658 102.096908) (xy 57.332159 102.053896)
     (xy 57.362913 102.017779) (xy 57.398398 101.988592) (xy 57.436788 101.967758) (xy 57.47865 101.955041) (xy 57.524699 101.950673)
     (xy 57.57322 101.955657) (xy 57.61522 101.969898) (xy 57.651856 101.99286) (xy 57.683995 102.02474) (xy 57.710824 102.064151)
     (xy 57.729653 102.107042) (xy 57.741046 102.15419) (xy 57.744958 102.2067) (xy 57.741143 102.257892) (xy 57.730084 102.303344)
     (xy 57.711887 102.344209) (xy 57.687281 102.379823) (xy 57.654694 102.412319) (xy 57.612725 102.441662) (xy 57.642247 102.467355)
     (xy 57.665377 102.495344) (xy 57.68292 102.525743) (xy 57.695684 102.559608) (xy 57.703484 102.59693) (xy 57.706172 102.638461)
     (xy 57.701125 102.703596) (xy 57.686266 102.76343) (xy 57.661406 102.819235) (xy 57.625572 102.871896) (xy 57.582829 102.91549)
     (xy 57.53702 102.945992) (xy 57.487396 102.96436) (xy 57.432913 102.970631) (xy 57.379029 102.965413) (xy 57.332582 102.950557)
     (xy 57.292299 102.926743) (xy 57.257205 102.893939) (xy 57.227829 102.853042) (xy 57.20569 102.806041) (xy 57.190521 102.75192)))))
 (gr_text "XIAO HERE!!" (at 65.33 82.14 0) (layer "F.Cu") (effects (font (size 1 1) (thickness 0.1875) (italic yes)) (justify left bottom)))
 (segment (start 79.24 104.12) (end 81.641 106.521) (width 0.2) (layer "B.Cu") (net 3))
 (segment (start 66.041 93.384) (end 66.041 105.399) (width 0.2) (layer "B.Cu") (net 3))
 (segment (start 60.83 107.89) (end 62.15 109.21) (width 0.2) (layer "B.Cu") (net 3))
 (segment (start 60.83 112.56) (end 62.15 111.24) (width 0.2) (layer "B.Cu") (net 3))
 (segment (start 62.15 111.24) (end 62.15 109.21) (width 0.2) (layer "B.Cu") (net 3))
 (segment (start 92.95 107.484816) (end 92.95 101.62) (width 0.2) (layer "B.Cu") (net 3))
 (segment (start 112.16 82.4) (end 77.705 82.4) (width 0.2) (layer "B.Cu") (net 3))
 (segment (start 66.041 105.399) (end 64.74 106.7) (width 0.2) (layer "B.Cu") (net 3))
 (segment (start 112.16 82.4) (end 112.16 101.62) (width 0.2) (layer "B.Cu") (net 3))
 (segment (start 60.83 106.75) (end 60.83 107.89) (width 0.2) (layer "B.Cu") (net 3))
 (segment (start 77.705 82.4) (end 77.365 82.06) (width 0.2) (layer "B.Cu") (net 3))
 (segment (start 64.66 106.7) (end 62.15 109.21) (width 0.2) (layer "B.Cu") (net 3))
 (segment (start 81.641 109.051) (end 91.383816 109.051) (width 0.2) (layer "B.Cu") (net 3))
 (segment (start 92.95 101.62) (end 112.16 101.62) (width 0.2) (layer "B.Cu") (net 3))
 (segment (start 66.041 93.384) (end 77.365 82.06) (width 0.2) (layer "B.Cu") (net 3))
 (segment (start 81.641 106.521) (end 81.641 109.051) (width 0.2) (layer "B.Cu") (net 3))
 (segment (start 91.383816 109.051) (end 92.95 107.484816) (width 0.2) (layer "B.Cu") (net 3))
 (segment (start 64.74 106.7) (end 64.66 106.7) (width 0.2) (layer "B.Cu") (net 3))
 (segment (start 63.303 93.582) (end 77.365 79.52) (width 0.2) (layer "B.Cu") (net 15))
 (segment (start 58.431 105.004) (end 63.303 100.132) (width 0.2) (layer "B.Cu") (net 15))
 (segment (start 58.431 109.709) (end 57.33 110.81) (width 0.2) (layer "B.Cu") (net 15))
 (segment (start 58.431 106.101) (end 58.431 109.709) (width 0.2) (layer "B.Cu") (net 15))
 (segment (start 57.33 105) (end 58.431 106.101) (width 0.2) (layer "B.Cu") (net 15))
 (segment (start 58.431 106.101) (end 58.431 105.004) (width 0.2) (layer "B.Cu") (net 15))
 (segment (start 63.303 100.132) (end 63.303 93.582) (width 0.2) (layer "B.Cu") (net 15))
 (segment (start 57.33 112.56) (end 55.431 110.661) (width 0.2) (layer "B.Cu") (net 7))
 (segment (start 55.431 110.661) (end 55.431 96.374) (width 0.2) (layer "B.Cu") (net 7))
 (segment (start 55.431 96.374) (end 62.125 89.68) (width 0.2) (layer "B.Cu") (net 7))
 (segment (start 80.08 94.76) (end 77.365 94.76) (width 0.2) (layer "B.Cu") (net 10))
 (segment (start 86.6 84.94) (end 86.6 88.24) (width 0.2) (layer "B.Cu") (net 10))
 (segment (start 86.6 88.24) (end 80.08 94.76) (width 0.2) (layer "B.Cu") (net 10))
 (segment (start 105.81 84.94) (end 88.581314 84.94) (width 0.2) (layer "B.Cu") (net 11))
 (segment (start 86.019686 83.539) (end 77.365 92.193686) (width 0.2) (layer "B.Cu") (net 11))
 (segment (start 88.581314 84.94) (end 87.180314 83.539) (width 0.2) (layer "B.Cu") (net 11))
 (segment (start 87.180314 83.539) (end 86.019686 83.539) (width 0.2) (layer "B.Cu") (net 11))
 (segment (start 77.365 92.193686) (end 77.365 92.22) (width 0.2) (layer "B.Cu") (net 11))
 (segment (start 86.6 98.08) (end 78.2 89.68) (width 0.2) (layer "F.Cu") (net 12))
 (segment (start 86.6 104.16) (end 86.6 98.08) (width 0.2) (layer "F.Cu") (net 12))
 (segment (start 83.29153 87.14) (end 78.2 87.14) (width 0.2) (layer "F.Cu") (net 13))
 (segment (start 100.31153 104.16) (end 83.29153 87.14) (width 0.2) (layer "F.Cu") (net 13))
 (segment (start 105.81 104.16) (end 100.31153 104.16) (width 0.2) (layer "F.Cu") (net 13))
 (segment (start 59.372 90.080626) (end 60.034374 90.743) (width 0.2) (layer "F.Cu") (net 2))
 (segment (start 62.56531 90.743) (end 63.439 91.61669) (width 0.2) (layer "F.Cu") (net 2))
 (segment (start 60.034374 90.743) (end 62.56531 90.743) (width 0.2) (layer "F.Cu") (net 2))
 (segment (start 62.125 82.06) (end 61.511374 82.06) (width 0.2) (layer "F.Cu") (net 2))
 (segment (start 59.372 84.199374) (end 59.372 90.080626) (width 0.2) (layer "F.Cu") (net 2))
 (segment (start 61.511374 82.06) (end 59.372 84.199374) (width 0.2) (layer "F.Cu") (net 2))
 (segment (start 63.439 91.61669) (end 63.439 107.899) (width 0.2) (layer "F.Cu") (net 2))
 (segment (start 63.439 107.899) (end 64.74 109.2) (width 0.2) (layer "F.Cu") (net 2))
 (segment (start 74.141 99.156) (end 74.141 104.101) (width 0.2) (layer "F.Cu") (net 5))
 (segment (start 62.125 87.14) (end 74.141 99.156) (width 0.2) (layer "F.Cu") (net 5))
 (segment (start 74.141 104.101) (end 79.24 109.2) (width 0.2) (layer "F.Cu") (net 5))
 (segment (start 59.773 86.338374) (end 61.511374 84.6) (width 0.2) (layer "F.Cu") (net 1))
 (segment (start 64.79559 90.43328) (end 62.56531 88.203) (width 0.2) (layer "F.Cu") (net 1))
 (segment (start 64.79559 90.43328) (end 64.74 90.48887) (width 0.2) (layer "F.Cu") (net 1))
 (segment (start 60.034374 88.203) (end 59.773 87.941626) (width 0.2) (layer "F.Cu") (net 1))
 (segment (start 61.511374 84.6) (end 62.125 84.6) (width 0.2) (layer "F.Cu") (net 1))
 (segment (start 64.74 104.12) (end 64.79559 104.06441) (width 0.2) (layer "F.Cu") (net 1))
 (segment (start 62.56531 88.203) (end 60.034374 88.203) (width 0.2) (layer "F.Cu") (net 1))
 (segment (start 64.74 90.48887) (end 64.74 104.2) (width 0.2) (layer "F.Cu") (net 1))
 (segment (start 59.773 87.941626) (end 59.773 86.338374) (width 0.2) (layer "F.Cu") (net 1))
 (segment (start 72.24 101.02) (end 72.22 101) (width 0.2) (layer "F.Cu") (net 4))
 (segment (start 72.24 101.1) (end 72.24 112.3) (width 0.2) (layer "B.Cu") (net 4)))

